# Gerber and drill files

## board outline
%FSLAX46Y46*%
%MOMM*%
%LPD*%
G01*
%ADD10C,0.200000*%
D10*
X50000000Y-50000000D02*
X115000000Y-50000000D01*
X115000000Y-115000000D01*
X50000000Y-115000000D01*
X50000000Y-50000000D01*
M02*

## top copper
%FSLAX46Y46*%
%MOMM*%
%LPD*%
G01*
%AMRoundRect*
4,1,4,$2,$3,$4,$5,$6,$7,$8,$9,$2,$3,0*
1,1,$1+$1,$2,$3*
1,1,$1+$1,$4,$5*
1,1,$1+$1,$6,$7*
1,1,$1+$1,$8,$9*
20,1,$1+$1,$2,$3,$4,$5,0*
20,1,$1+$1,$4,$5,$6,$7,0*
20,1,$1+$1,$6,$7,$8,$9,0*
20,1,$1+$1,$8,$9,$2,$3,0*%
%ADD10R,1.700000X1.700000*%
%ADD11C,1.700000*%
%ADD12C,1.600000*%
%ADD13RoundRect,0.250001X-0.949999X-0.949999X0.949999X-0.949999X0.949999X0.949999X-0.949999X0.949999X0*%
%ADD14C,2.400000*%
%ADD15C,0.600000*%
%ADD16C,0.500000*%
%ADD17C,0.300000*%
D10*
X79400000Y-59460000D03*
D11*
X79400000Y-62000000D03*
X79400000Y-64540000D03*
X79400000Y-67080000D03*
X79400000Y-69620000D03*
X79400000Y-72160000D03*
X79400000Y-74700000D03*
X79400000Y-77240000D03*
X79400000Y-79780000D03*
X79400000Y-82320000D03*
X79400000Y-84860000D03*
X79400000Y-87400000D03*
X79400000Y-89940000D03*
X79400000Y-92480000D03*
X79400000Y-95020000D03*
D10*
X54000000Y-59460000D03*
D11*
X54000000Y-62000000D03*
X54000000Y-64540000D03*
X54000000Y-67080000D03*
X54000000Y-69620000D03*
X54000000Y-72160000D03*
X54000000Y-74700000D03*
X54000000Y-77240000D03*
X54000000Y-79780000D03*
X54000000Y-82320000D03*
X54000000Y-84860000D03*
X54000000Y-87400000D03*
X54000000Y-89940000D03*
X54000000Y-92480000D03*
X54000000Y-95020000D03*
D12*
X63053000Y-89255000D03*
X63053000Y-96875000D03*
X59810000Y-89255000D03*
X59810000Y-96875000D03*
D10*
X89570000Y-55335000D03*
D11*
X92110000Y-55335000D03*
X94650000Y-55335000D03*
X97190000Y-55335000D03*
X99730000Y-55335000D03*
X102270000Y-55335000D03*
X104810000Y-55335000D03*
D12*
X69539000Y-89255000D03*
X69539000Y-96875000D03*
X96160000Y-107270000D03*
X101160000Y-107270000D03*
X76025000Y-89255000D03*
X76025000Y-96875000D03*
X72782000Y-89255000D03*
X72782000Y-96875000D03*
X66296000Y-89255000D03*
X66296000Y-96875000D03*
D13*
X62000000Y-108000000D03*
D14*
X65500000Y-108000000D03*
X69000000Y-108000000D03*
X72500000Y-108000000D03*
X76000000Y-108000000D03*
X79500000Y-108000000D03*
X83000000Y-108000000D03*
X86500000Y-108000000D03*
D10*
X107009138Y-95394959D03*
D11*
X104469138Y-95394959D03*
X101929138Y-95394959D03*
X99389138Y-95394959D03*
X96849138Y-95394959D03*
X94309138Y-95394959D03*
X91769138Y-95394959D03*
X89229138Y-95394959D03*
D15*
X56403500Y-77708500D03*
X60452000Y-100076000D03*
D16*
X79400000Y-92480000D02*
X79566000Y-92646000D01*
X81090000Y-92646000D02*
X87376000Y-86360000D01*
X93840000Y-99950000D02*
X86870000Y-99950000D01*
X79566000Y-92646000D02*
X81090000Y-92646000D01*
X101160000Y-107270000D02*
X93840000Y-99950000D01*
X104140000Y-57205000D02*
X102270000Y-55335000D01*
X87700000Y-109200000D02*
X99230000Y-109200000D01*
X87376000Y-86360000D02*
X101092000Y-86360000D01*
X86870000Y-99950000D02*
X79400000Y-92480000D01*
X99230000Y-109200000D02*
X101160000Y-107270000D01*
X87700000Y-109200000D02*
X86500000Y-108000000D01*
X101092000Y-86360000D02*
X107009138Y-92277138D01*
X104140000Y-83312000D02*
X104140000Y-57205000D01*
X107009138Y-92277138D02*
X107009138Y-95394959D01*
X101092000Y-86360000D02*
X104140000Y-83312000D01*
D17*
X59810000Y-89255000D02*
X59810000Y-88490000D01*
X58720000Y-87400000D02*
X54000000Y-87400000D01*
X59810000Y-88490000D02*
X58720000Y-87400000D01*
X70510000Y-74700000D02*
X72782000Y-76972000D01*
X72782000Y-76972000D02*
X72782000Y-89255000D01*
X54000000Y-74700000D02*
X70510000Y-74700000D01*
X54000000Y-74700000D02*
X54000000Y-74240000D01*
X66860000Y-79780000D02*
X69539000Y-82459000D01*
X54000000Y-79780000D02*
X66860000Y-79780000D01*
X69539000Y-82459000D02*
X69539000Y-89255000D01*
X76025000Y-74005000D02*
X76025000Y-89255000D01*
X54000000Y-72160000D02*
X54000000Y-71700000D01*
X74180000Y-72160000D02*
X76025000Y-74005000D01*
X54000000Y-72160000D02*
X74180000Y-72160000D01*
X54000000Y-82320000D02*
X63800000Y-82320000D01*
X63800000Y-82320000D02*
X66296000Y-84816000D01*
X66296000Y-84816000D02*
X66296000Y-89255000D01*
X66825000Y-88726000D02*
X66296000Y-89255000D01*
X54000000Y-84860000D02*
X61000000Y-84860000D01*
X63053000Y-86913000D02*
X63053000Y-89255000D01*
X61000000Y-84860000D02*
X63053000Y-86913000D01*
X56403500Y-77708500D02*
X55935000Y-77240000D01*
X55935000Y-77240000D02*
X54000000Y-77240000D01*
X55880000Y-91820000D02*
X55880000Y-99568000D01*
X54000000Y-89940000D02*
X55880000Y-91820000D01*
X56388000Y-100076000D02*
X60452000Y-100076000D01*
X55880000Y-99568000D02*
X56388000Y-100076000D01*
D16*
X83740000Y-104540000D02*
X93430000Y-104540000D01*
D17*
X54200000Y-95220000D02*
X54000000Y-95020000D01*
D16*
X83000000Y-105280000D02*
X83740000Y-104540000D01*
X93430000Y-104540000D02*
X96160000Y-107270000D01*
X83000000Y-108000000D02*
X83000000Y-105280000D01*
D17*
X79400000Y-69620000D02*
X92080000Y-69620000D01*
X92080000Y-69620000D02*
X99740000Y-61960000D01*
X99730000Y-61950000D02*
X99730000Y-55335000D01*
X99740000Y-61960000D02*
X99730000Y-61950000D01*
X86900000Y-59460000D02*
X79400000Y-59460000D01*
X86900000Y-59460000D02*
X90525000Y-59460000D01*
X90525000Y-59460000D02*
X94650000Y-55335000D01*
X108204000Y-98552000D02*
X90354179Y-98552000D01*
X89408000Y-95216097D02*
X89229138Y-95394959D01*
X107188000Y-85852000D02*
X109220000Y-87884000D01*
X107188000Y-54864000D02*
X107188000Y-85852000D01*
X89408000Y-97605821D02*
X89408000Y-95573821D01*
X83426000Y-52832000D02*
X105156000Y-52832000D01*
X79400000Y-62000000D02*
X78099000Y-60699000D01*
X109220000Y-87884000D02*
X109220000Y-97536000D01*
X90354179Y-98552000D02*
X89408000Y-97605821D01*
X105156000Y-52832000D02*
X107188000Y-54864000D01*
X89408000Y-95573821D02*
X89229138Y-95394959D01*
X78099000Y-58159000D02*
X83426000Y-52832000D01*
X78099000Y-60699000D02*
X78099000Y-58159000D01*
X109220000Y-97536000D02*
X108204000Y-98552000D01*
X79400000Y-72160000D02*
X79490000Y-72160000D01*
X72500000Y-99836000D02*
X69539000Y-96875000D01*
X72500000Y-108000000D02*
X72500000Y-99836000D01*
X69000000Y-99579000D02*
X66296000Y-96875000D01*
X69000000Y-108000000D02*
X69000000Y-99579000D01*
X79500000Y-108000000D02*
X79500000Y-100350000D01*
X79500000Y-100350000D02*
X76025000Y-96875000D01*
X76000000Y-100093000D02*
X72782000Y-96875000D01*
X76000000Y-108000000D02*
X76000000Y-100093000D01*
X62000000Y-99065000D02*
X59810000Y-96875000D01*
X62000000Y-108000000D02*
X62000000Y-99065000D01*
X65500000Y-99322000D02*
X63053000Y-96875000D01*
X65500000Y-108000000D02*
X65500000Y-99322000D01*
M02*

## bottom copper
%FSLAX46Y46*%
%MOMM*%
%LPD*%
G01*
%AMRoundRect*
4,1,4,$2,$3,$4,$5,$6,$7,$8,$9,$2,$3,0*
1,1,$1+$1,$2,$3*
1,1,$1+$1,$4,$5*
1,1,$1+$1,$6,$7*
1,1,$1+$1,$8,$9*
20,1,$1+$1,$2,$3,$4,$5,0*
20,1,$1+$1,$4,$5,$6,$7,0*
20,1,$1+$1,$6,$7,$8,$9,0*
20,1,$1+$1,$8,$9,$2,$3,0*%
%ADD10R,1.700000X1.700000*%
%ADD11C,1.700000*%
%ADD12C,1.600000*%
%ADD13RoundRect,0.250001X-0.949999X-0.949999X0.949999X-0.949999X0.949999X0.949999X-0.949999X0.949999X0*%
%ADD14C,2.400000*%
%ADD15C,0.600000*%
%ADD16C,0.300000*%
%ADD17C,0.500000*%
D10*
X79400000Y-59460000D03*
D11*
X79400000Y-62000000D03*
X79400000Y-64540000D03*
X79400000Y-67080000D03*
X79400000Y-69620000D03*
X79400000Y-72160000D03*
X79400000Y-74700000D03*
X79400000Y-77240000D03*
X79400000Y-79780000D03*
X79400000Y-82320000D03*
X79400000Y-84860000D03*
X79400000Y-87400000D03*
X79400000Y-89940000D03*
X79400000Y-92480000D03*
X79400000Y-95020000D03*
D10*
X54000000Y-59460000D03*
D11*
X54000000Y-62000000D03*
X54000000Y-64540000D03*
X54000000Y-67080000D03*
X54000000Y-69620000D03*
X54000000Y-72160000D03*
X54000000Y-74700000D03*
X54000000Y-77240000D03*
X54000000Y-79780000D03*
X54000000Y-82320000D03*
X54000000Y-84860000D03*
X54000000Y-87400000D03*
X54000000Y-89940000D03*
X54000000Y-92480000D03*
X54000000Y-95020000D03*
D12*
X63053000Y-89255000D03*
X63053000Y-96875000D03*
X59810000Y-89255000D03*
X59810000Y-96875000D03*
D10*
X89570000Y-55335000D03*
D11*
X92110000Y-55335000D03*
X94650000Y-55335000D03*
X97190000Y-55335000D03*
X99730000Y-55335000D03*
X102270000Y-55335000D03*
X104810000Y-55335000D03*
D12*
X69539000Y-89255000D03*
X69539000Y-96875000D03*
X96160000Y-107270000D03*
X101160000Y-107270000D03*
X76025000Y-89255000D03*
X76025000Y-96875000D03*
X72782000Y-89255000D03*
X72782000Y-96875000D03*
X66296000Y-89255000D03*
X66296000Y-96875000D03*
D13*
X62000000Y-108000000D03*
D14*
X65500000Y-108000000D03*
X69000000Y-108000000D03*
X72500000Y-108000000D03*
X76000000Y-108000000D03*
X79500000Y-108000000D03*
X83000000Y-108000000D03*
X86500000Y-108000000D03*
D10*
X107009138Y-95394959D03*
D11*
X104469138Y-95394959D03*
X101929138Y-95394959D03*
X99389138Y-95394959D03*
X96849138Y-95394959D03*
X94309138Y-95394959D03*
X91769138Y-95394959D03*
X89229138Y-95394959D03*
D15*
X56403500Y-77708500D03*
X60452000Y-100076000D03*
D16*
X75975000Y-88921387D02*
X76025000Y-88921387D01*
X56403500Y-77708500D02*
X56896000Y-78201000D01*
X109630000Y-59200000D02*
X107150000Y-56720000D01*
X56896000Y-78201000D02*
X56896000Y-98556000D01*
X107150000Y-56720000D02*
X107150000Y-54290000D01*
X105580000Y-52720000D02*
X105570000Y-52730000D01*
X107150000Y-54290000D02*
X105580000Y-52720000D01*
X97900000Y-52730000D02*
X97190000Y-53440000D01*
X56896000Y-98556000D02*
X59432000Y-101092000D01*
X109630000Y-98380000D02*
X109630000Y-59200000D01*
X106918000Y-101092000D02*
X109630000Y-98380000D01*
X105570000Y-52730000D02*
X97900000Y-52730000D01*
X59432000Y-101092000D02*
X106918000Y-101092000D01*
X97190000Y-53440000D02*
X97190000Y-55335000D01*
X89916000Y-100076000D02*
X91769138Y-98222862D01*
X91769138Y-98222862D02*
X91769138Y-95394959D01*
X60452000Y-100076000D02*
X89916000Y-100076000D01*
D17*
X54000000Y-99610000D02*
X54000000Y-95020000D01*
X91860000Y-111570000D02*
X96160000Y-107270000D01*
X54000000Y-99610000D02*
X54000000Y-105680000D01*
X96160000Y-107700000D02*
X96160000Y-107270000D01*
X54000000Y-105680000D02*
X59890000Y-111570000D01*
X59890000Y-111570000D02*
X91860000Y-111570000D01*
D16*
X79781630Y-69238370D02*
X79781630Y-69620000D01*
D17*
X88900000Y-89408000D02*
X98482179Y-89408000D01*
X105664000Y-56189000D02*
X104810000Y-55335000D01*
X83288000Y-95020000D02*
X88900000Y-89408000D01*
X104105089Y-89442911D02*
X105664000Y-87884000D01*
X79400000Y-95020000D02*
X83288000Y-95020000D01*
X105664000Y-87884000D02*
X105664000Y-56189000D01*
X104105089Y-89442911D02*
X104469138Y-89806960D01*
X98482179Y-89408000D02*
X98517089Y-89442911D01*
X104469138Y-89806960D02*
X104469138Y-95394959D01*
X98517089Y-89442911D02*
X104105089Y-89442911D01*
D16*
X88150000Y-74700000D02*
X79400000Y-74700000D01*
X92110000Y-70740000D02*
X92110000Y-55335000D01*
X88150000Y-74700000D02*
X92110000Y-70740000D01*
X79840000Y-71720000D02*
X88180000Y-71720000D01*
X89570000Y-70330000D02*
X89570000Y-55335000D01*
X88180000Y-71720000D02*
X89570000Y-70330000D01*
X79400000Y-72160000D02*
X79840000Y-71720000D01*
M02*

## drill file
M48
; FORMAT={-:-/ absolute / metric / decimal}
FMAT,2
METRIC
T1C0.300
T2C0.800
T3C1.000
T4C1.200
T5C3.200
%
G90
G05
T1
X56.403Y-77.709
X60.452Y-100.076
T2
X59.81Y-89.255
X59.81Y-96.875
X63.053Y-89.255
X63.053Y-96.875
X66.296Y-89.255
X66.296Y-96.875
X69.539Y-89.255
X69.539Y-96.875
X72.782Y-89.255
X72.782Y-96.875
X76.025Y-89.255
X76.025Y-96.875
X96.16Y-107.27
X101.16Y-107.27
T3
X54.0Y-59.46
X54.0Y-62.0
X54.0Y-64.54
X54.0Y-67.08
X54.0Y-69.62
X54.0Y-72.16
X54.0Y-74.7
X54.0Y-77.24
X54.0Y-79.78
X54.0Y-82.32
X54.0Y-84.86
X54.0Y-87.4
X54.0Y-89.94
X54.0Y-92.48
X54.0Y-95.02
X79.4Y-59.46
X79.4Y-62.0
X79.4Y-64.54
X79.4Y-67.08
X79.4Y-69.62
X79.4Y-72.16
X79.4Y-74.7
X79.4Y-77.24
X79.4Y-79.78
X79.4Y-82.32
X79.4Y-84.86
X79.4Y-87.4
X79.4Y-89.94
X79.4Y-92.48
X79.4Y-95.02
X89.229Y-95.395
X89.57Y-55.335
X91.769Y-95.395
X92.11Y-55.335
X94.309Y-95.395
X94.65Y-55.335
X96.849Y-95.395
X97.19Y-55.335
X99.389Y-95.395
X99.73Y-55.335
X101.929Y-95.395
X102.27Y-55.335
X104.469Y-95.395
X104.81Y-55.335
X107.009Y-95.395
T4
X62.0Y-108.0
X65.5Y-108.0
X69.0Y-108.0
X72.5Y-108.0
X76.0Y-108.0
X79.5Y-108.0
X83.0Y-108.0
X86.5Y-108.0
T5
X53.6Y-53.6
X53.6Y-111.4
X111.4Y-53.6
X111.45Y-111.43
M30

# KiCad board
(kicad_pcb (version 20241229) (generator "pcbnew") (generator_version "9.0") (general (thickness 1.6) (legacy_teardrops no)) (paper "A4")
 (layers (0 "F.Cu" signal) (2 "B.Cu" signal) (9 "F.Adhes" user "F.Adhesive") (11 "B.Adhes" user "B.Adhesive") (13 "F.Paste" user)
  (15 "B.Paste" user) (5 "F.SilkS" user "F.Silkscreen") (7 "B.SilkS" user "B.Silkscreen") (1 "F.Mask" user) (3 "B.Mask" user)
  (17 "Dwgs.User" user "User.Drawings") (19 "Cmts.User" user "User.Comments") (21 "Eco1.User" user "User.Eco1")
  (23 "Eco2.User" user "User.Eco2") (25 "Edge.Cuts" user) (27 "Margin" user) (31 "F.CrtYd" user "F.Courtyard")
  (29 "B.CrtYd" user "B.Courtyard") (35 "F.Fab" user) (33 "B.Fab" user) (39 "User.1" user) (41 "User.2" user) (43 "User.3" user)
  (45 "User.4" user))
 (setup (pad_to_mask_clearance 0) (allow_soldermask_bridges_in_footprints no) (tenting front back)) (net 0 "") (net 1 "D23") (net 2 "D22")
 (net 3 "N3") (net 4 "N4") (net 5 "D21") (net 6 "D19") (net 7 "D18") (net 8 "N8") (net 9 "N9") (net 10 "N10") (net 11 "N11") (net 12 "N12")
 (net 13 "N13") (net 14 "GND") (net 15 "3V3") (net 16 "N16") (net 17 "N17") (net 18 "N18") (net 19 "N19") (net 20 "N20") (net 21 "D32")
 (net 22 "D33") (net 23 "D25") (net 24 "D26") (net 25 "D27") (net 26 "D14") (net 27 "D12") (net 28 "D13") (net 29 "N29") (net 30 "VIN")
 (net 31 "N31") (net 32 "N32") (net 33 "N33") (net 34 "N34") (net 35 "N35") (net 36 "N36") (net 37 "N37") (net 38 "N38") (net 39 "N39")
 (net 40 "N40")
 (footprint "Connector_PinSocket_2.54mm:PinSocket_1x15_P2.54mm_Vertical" (layer "F.Cu") (at 79.4 59.46)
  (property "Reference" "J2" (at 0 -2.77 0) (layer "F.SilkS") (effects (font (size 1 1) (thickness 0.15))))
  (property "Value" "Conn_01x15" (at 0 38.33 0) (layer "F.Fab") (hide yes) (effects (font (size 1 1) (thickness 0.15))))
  (pad "1" thru_hole rect (at 0 0) (size 1.7 1.7) (drill 1) (layers "*.Cu" "*.Mask") (remove_unused_layers no) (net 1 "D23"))
  (pad "2" thru_hole circle (at 0 2.54) (size 1.7 1.7) (drill 1) (layers "*.Cu" "*.Mask") (remove_unused_layers no) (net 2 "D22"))
  (pad "3" thru_hole circle (at 0 5.08) (size 1.7 1.7) (drill 1) (layers "*.Cu" "*.Mask") (remove_unused_layers no) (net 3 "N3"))
  (pad "4" thru_hole circle (at 0 7.62) (size 1.7 1.7) (drill 1) (layers "*.Cu" "*.Mask") (remove_unused_layers no) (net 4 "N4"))
  (pad "5" thru_hole circle (at 0 10.16) (size 1.7 1.7) (drill 1) (layers "*.Cu" "*.Mask") (remove_unused_layers no) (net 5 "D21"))
  (pad "6" thru_hole circle (at 0 12.7) (size 1.7 1.7) (drill 1) (layers "*.Cu" "*.Mask") (remove_unused_layers no) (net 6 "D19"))
  (pad "7" thru_hole circle (at 0 15.24) (size 1.7 1.7) (drill 1) (layers "*.Cu" "*.Mask") (remove_unused_layers no) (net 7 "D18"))
  (pad "8" thru_hole circle (at 0 17.78) (size 1.7 1.7) (drill 1) (layers "*.Cu" "*.Mask") (remove_unused_layers no) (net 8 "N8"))
  (pad "9" thru_hole circle (at 0 20.32) (size 1.7 1.7) (drill 1) (layers "*.Cu" "*.Mask") (remove_unused_layers no) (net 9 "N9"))
  (pad "10" thru_hole circle (at 0 22.86) (size 1.7 1.7) (drill 1) (layers "*.Cu" "*.Mask") (remove_unused_layers no) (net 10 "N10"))
  (pad "11" thru_hole circle (at 0 25.4) (size 1.7 1.7) (drill 1) (layers "*.Cu" "*.Mask") (remove_unused_layers no) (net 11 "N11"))
  (pad "12" thru_hole circle (at 0 27.94) (size 1.7 1.7) (drill 1) (layers "*.Cu" "*.Mask") (remove_unused_layers no) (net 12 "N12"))
  (pad "13" thru_hole circle (at 0 30.48) (size 1.7 1.7) (drill 1) (layers "*.Cu" "*.Mask") (remove_unused_layers no) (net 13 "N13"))
  (pad "14" thru_hole circle (at 0 33.02) (size 1.7 1.7) (drill 1) (layers "*.Cu" "*.Mask") (remove_unused_layers no) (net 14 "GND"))
  (pad "15" thru_hole circle (at 0 35.56) (size 1.7 1.7) (drill 1) (layers "*.Cu" "*.Mask") (remove_unused_layers no) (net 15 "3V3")))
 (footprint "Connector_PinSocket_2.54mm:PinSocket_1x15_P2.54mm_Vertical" (layer "F.Cu") (at 54 59.46)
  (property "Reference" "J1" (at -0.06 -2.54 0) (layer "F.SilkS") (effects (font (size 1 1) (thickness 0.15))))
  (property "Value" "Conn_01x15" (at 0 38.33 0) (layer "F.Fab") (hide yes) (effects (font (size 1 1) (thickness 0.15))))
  (pad "1" thru_hole rect (at 0 0) (size 1.7 1.7) (drill 1) (layers "*.Cu" "*.Mask") (remove_unused_layers no) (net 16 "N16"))
  (pad "2" thru_hole circle (at 0 2.54) (size 1.7 1.7) (drill 1) (layers "*.Cu" "*.Mask") (remove_unused_layers no) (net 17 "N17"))
  (pad "3" thru_hole circle (at 0 5.08) (size 1.7 1.7) (drill 1) (layers "*.Cu" "*.Mask") (remove_unused_layers no) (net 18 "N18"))
  (pad "4" thru_hole circle (at 0 7.62) (size 1.7 1.7) (drill 1) (layers "*.Cu" "*.Mask") (remove_unused_layers no) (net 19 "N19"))
  (pad "5" thru_hole circle (at 0 10.16) (size 1.7 1.7) (drill 1) (layers "*.Cu" "*.Mask") (remove_unused_layers no) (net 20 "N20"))
  (pad "6" thru_hole circle (at 0 12.7) (size 1.7 1.7) (drill 1) (layers "*.Cu" "*.Mask") (remove_unused_layers no) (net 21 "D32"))
  (pad "7" thru_hole circle (at 0 15.24) (size 1.7 1.7) (drill 1) (layers "*.Cu" "*.Mask") (remove_unused_layers no) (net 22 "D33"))
  (pad "8" thru_hole circle (at 0 17.78) (size 1.7 1.7) (drill 1) (layers "*.Cu" "*.Mask") (remove_unused_layers no) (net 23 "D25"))
  (pad "9" thru_hole circle (at 0 20.32) (size 1.7 1.7) (drill 1) (layers "*.Cu" "*.Mask") (remove_unused_layers no) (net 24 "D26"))
  (pad "10" thru_hole circle (at 0 22.86) (size 1.7 1.7) (drill 1) (layers "*.Cu" "*.Mask") (remove_unused_layers no) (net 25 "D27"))
  (pad "11" thru_hole circle (at 0 25.4) (size 1.7 1.7) (drill 1) (layers "*.Cu" "*.Mask") (remove_unused_layers no) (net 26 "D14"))
  (pad "12" thru_hole circle (at 0 27.94) (size 1.7 1.7) (drill 1) (layers "*.Cu" "*.Mask") (remove_unused_layers no) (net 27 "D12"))
  (pad "13" thru_hole circle (at 0 30.48) (size 1.7 1.7) (drill 1) (layers "*.Cu" "*.Mask") (remove_unused_layers no) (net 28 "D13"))
  (pad "14" thru_hole circle (at 0 33.02) (size 1.7 1.7) (drill 1) (layers "*.Cu" "*.Mask") (remove_unused_layers no) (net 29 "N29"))
  (pad "15" thru_hole circle (at 0 35.56) (size 1.7 1.7) (drill 1) (layers "*.Cu" "*.Mask") (remove_unused_layers no) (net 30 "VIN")))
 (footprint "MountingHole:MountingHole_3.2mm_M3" (layer "F.Cu") (at 53.6 53.6)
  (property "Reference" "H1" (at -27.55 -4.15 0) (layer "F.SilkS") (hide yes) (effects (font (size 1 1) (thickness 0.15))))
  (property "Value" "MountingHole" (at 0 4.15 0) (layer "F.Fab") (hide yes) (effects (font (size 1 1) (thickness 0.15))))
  (pad "" np_thru_hole circle (at 0 0) (size 3.2 3.2) (drill 3.2) (layers "*.Cu" "*.Mask")))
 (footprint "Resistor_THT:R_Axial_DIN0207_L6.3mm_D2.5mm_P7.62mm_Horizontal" (layer "F.Cu") (at 63.053 89.255 -90)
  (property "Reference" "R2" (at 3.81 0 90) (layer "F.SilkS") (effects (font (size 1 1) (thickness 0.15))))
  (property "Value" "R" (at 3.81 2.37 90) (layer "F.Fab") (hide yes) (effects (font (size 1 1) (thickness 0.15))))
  (pad "1" thru_hole circle (at 0 0 270) (size 1.6 1.6) (drill 0.8) (layers "*.Cu" "*.Mask") (remove_unused_layers no) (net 26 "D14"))
  (pad "2" thru_hole circle (at 7.62 0 270) (size 1.6 1.6) (drill 0.8) (layers "*.Cu" "*.Mask") (remove_unused_layers no) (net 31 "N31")))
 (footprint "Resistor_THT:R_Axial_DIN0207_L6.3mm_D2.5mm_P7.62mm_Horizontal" (layer "F.Cu") (at 59.81 89.255 -90)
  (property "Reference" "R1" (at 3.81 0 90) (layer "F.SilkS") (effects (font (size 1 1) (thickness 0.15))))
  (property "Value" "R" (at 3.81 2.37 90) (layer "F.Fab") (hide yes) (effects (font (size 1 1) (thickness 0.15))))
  (pad "1" thru_hole circle (at 0 0 270) (size 1.6 1.6) (drill 0.8) (layers "*.Cu" "*.Mask") (remove_unused_layers no) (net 27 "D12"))
  (pad "2" thru_hole circle (at 7.62 0 270) (size 1.6 1.6) (drill 0.8) (layers "*.Cu" "*.Mask") (remove_unused_layers no) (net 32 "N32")))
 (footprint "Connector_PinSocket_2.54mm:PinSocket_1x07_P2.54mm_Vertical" (layer "F.Cu") (at 89.57 55.335 90)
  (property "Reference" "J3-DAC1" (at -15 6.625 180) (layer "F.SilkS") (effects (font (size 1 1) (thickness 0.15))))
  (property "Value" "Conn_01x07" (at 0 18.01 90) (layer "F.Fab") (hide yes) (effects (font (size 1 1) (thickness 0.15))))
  (pad "1" thru_hole rect (at 0 0 90) (size 1.7 1.7) (drill 1) (layers "*.Cu" "*.Mask") (remove_unused_layers no) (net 6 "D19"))
  (pad "2" thru_hole circle (at 0 2.54 90) (size 1.7 1.7) (drill 1) (layers "*.Cu" "*.Mask") (remove_unused_layers no) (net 7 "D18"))
  (pad "3" thru_hole circle (at 0 5.08 90) (size 1.7 1.7) (drill 1) (layers "*.Cu" "*.Mask") (remove_unused_layers no) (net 1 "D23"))
  (pad "4" thru_hole circle (at 0 7.62 90) (size 1.7 1.7) (drill 1) (layers "*.Cu" "*.Mask") (remove_unused_layers no) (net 23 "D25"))
  (pad "5" thru_hole circle (at 0 10.16 90) (size 1.7 1.7) (drill 1) (layers "*.Cu" "*.Mask") (remove_unused_layers no) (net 5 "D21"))
  (pad "6" thru_hole circle (at 0 12.7 90) (size 1.7 1.7) (drill 1) (layers "*.Cu" "*.Mask") (remove_unused_layers no) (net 14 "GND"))
  (pad "7" thru_hole circle (at 0 15.24 90) (size 1.7 1.7) (drill 1) (layers "*.Cu" "*.Mask") (remove_unused_layers no) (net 15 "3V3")))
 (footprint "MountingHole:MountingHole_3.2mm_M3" (layer "F.Cu") (at 53.6 111.4)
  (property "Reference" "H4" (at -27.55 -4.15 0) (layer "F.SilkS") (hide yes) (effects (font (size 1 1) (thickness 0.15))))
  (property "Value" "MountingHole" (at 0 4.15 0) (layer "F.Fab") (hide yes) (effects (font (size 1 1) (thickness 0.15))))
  (pad "" np_thru_hole circle (at 0 0) (size 3.2 3.2) (drill 3.2) (layers "*.Cu" "*.Mask")))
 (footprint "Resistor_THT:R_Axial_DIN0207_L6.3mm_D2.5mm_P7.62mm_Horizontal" (layer "F.Cu") (at 69.539 89.255 -90)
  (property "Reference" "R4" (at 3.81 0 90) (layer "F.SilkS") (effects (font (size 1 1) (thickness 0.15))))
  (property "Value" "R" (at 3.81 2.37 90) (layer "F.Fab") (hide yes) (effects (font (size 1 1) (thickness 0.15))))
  (pad "1" thru_hole circle (at 0 0 270) (size 1.6 1.6) (drill 0.8) (layers "*.Cu" "*.Mask") (remove_unused_layers no) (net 24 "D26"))
  (pad "2" thru_hole circle (at 7.62 0 270) (size 1.6 1.6) (drill 0.8) (layers "*.Cu" "*.Mask") (remove_unused_layers no) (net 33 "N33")))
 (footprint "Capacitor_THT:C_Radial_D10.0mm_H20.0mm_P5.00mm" (layer "F.Cu") (at 96.16 107.27)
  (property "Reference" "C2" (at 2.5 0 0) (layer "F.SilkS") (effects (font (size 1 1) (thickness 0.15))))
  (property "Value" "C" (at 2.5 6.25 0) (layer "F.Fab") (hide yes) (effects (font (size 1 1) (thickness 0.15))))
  (pad "1" thru_hole circle (at 0 0) (size 1.6 1.6) (drill 0.8) (layers "*.Cu" "*.Mask") (remove_unused_layers no) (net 30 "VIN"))
  (pad "2" thru_hole circle (at 5 0) (size 1.6 1.6) (drill 0.8) (layers "*.Cu" "*.Mask") (remove_unused_layers no) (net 14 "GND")))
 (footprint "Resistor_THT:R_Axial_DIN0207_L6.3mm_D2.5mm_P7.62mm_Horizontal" (layer "F.Cu") (at 76.025 89.255 -90)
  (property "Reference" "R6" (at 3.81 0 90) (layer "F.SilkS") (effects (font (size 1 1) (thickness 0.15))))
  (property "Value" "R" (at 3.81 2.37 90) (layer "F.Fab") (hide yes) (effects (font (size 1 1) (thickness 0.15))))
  (pad "1" thru_hole circle (at 0 0 270) (size 1.6 1.6) (drill 0.8) (layers "*.Cu" "*.Mask") (remove_unused_layers no) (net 21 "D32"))
  (pad "2" thru_hole circle (at 7.62 0 270) (size 1.6 1.6) (drill 0.8) (layers "*.Cu" "*.Mask") (remove_unused_layers no) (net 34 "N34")))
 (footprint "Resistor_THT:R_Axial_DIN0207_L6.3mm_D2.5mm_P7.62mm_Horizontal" (layer "F.Cu") (at 72.782 89.255 -90)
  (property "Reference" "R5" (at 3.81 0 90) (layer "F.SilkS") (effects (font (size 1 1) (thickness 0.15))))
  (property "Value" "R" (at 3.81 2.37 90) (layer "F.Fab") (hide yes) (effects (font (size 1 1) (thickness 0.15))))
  (pad "1" thru_hole circle (at 0 0 270) (size 1.6 1.6) (drill 0.8) (layers "*.Cu" "*.Mask") (remove_unused_layers no) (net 22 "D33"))
  (pad "2" thru_hole circle (at 7.62 0 270) (size 1.6 1.6) (drill 0.8) (layers "*.Cu" "*.Mask") (remove_unused_layers no) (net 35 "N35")))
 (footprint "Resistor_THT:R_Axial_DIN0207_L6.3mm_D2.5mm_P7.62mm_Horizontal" (layer "F.Cu") (at 66.296 89.255 -90)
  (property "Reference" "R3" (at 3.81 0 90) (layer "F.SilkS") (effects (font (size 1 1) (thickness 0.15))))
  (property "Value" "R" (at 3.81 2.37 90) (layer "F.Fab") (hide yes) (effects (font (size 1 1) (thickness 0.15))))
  (pad "1" thru_hole circle (at 0 0 270) (size 1.6 1.6) (drill 0.8) (layers "*.Cu" "*.Mask") (remove_unused_layers no) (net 25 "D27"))
  (pad "2" thru_hole circle (at 7.62 0 270) (size 1.6 1.6) (drill 0.8) (layers "*.Cu" "*.Mask") (remove_unused_layers no) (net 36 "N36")))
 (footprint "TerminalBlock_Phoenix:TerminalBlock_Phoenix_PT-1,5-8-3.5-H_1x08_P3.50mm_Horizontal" (layer "F.Cu") (at 62 108)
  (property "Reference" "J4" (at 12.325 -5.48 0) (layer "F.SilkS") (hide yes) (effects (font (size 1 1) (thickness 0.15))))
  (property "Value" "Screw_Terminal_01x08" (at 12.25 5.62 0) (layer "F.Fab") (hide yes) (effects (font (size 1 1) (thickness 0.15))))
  (pad "1" thru_hole roundrect (at 0 0) (size 2.4 2.4) (drill 1.2) (layers "*.Cu" "*.Mask") (remove_unused_layers no)
   (roundrect_rratio 0.104167) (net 32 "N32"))
  (pad "2" thru_hole circle (at 3.5 0) (size 2.4 2.4) (drill 1.2) (layers "*.Cu" "*.Mask") (remove_unused_layers no) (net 31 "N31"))
  (pad "3" thru_hole circle (at 7 0) (size 2.4 2.4) (drill 1.2) (layers "*.Cu" "*.Mask") (remove_unused_layers no) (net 36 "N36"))
  (pad "4" thru_hole circle (at 10.5 0) (size 2.4 2.4) (drill 1.2) (layers "*.Cu" "*.Mask") (remove_unused_layers no) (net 33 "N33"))
  (pad "5" thru_hole circle (at 14 0) (size 2.4 2.4) (drill 1.2) (layers "*.Cu" "*.Mask") (remove_unused_layers no) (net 35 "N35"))
  (pad "6" thru_hole circle (at 17.5 0) (size 2.4 2.4) (drill 1.2) (layers "*.Cu" "*.Mask") (remove_unused_layers no) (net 34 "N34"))
  (pad "7" thru_hole circle (at 21 0) (size 2.4 2.4) (drill 1.2) (layers "*.Cu" "*.Mask") (remove_unused_layers no) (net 30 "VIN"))
  (pad "8" thru_hole circle (at 24.5 0) (size 2.4 2.4) (drill 1.2) (layers "*.Cu" "*.Mask") (remove_unused_layers no) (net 14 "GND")))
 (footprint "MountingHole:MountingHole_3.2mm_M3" (layer "F.Cu") (at 111.45 111.43)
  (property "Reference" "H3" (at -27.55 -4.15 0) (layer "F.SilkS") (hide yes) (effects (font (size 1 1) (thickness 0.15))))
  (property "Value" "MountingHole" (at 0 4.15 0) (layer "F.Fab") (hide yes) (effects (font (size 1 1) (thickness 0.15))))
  (pad "" np_thru_hole circle (at 0 0) (size 3.2 3.2) (drill 3.2) (layers "*.Cu" "*.Mask")))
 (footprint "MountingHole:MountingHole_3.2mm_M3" (layer "F.Cu") (at 111.4 53.6)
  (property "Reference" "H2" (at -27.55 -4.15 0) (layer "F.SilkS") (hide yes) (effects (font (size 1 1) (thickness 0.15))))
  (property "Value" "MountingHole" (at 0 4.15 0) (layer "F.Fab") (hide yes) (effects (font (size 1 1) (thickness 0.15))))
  (pad "" np_thru_hole circle (at 0 0) (size 3.2 3.2) (drill 3.2) (layers "*.Cu" "*.Mask")))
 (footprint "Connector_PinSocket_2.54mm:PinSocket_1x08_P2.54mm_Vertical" (layer "F.Cu") (at 107.009138 95.394959 -90)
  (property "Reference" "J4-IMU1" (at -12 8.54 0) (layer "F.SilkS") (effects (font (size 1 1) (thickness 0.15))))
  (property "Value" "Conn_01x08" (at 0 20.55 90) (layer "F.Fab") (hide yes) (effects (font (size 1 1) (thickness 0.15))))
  (pad "1" thru_hole rect (at 0 0 270) (size 1.7 1.7) (drill 1) (layers "*.Cu" "*.Mask") (remove_unused_layers no) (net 14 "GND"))
  (pad "2" thru_hole circle (at 0 2.54 270) (size 1.7 1.7) (drill 1) (layers "*.Cu" "*.Mask") (remove_unused_layers no) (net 15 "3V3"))
  (pad "3" thru_hole circle (at 0 5.08 270) (size 1.7 1.7) (drill 1) (layers "*.Cu" "*.Mask") (remove_unused_layers no) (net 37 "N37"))
  (pad "4" thru_hole circle (at 0 7.62 270) (size 1.7 1.7) (drill 1) (layers "*.Cu" "*.Mask") (remove_unused_layers no) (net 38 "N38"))
  (pad "5" thru_hole circle (at 0 10.16 270) (size 1.7 1.7) (drill 1) (layers "*.Cu" "*.Mask") (remove_unused_layers no) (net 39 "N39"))
  (pad "6" thru_hole circle (at 0 12.7 270) (size 1.7 1.7) (drill 1) (layers "*.Cu" "*.Mask") (remove_unused_layers no) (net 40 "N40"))
  (pad "7" thru_hole circle (at 0 15.24 270) (size 1.7 1.7) (drill 1) (layers "*.Cu" "*.Mask") (remove_unused_layers no) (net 28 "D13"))
  (pad "8" thru_hole circle (at 0 17.78 270) (size 1.7 1.7) (drill 1) (layers "*.Cu" "*.Mask") (remove_unused_layers no) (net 2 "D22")))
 (gr_rect (start 50 50) (end 115 115) (stroke (width 0.2) (type solid)) (fill no) (layer "Edge.Cuts"))
 (segment (start 79.4 92.48) (end 79.566 92.646) (width 0.5) (layer "F.Cu") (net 14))
 (segment (start 81.09 92.646) (end 87.376 86.36) (width 0.5) (layer "F.Cu") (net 14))
 (segment (start 93.84 99.95) (end 86.87 99.95) (width 0.5) (layer "F.Cu") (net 14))
 (segment (start 79.566 92.646) (end 81.09 92.646) (width 0.5) (layer "F.Cu") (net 14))
 (segment (start 101.16 107.27) (end 93.84 99.95) (width 0.5) (layer "F.Cu") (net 14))
 (segment (start 104.14 57.205) (end 102.27 55.335) (width 0.5) (layer "F.Cu") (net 14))
 (segment (start 87.7 109.2) (end 99.23 109.2) (width 0.5) (layer "F.Cu") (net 14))
 (segment (start 87.376 86.36) (end 101.092 86.36) (width 0.5) (layer "F.Cu") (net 14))
 (segment (start 86.87 99.95) (end 79.4 92.48) (width 0.5) (layer "F.Cu") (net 14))
 (segment (start 99.23 109.2) (end 101.16 107.27) (width 0.5) (layer "F.Cu") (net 14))
 (segment (start 87.7 109.2) (end 86.5 108) (width 0.5) (layer "F.Cu") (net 14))
 (segment (start 101.092 86.36) (end 107.009138 92.277138) (width 0.5) (layer "F.Cu") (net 14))
 (segment (start 104.14 83.312) (end 104.14 57.205) (width 0.5) (layer "F.Cu") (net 14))
 (segment (start 107.009138 92.277138) (end 107.009138 95.394959) (width 0.5) (layer "F.Cu") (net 14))
 (segment (start 101.092 86.36) (end 104.14 83.312) (width 0.5) (layer "F.Cu") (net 14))
 (segment (start 59.81 89.255) (end 59.81 88.49) (width 0.3) (layer "F.Cu") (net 27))
 (segment (start 58.72 87.4) (end 54 87.4) (width 0.3) (layer "F.Cu") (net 27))
 (segment (start 59.81 88.49) (end 58.72 87.4) (width 0.3) (layer "F.Cu") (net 27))
 (segment (start 70.51 74.7) (end 72.782 76.972) (width 0.3) (layer "F.Cu") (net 22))
 (segment (start 72.782 76.972) (end 72.782 89.255) (width 0.3) (layer "F.Cu") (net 22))
 (segment (start 54 74.7) (end 70.51 74.7) (width 0.3) (layer "F.Cu") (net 22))
 (segment (start 54 74.7) (end 54 74.24) (width 0.3) (layer "F.Cu") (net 22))
 (segment (start 66.86 79.78) (end 69.539 82.459) (width 0.3) (layer "F.Cu") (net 24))
 (segment (start 54 79.78) (end 66.86 79.78) (width 0.3) (layer "F.Cu") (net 24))
 (segment (start 69.539 82.459) (end 69.539 89.255) (width 0.3) (layer "F.Cu") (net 24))
 (segment (start 76.025 74.005) (end 76.025 89.255) (width 0.3) (layer "F.Cu") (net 21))
 (segment (start 54 72.16) (end 54 71.7) (width 0.3) (layer "F.Cu") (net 21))
 (segment (start 74.18 72.16) (end 76.025 74.005) (width 0.3) (layer "F.Cu") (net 21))
 (segment (start 54 72.16) (end 74.18 72.16) (width 0.3) (layer "F.Cu") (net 21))
 (segment (start 75.975 88.921387) (end 76.025 88.921387) (width 0.3) (layer "B.Cu") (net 21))
 (segment (start 54 82.32) (end 63.8 82.32) (width 0.3) (layer "F.Cu") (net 25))
 (segment (start 63.8 82.32) (end 66.296 84.816) (width 0.3) (layer "F.Cu") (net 25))
 (segment (start 66.296 84.816) (end 66.296 89.255) (width 0.3) (layer "F.Cu") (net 25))
 (segment (start 66.825 88.726) (end 66.296 89.255) (width 0.3) (layer "F.Cu") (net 25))
 (segment (start 54 84.86) (end 61 84.86) (width 0.3) (layer "F.Cu") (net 26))
 (segment (start 63.053 86.913) (end 63.053 89.255) (width 0.3) (layer "F.Cu") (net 26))
 (segment (start 61 84.86) (end 63.053 86.913) (width 0.3) (layer "F.Cu") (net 26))
 (segment (start 56.4035 77.7085) (end 55.935 77.24) (width 0.3) (layer "F.Cu") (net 23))
 (segment (start 55.935 77.24) (end 54 77.24) (width 0.3) (layer "F.Cu") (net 23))
 (via (at 56.4035 77.7085) (size 0.6) (drill 0.3) (layers "F.Cu" "B.Cu") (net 23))
 (segment (start 56.4035 77.7085) (end 56.896 78.201) (width 0.3) (layer "B.Cu") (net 23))
 (segment (start 109.63 59.2) (end 107.15 56.72) (width 0.3) (layer "B.Cu") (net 23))
 (segment (start 56.896 78.201) (end 56.896 98.556) (width 0.3) (layer "B.Cu") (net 23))
 (segment (start 107.15 56.72) (end 107.15 54.29) (width 0.3) (layer "B.Cu") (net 23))
 (segment (start 105.58 52.72) (end 105.57 52.73) (width 0.3) (layer "B.Cu") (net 23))
 (segment (start 107.15 54.29) (end 105.58 52.72) (width 0.3) (layer "B.Cu") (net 23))
 (segment (start 97.9 52.73) (end 97.19 53.44) (width 0.3) (layer "B.Cu") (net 23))
 (segment (start 56.896 98.556) (end 59.432 101.092) (width 0.3) (layer "B.Cu") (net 23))
 (segment (start 109.63 98.38) (end 109.63 59.2) (width 0.3) (layer "B.Cu") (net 23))
 (segment (start 106.918 101.092) (end 109.63 98.38) (width 0.3) (layer "B.Cu") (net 23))
 (segment (start 105.57 52.73) (end 97.9 52.73) (width 0.3) (layer "B.Cu") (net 23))
 (segment (start 59.432 101.092) (end 106.918 101.092) (width 0.3) (layer "B.Cu") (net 23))
 (segment (start 97.19 53.44) (end 97.19 55.335) (width 0.3) (layer "B.Cu") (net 23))
 (segment (start 55.88 91.82) (end 55.88 99.568) (width 0.3) (layer "F.Cu") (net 28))
 (segment (start 54 89.94) (end 55.88 91.82) (width 0.3) (layer "F.Cu") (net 28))
 (segment (start 56.388 100.076) (end 60.452 100.076) (width 0.3) (layer "F.Cu") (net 28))
 (segment (start 55.88 99.568) (end 56.388 100.076) (width 0.3) (layer "F.Cu") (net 28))
 (via (at 60.452 100.076) (size 0.6) (drill 0.3) (layers "F.Cu" "B.Cu") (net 28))
 (segment (start 89.916 100.076) (end 91.769138 98.222862) (width 0.3) (layer "B.Cu") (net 28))
 (segment (start 91.769138 98.222862) (end 91.769138 95.394959) (width 0.3) (layer "B.Cu") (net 28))
 (segment (start 60.452 100.076) (end 89.916 100.076) (width 0.3) (layer "B.Cu") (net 28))
 (segment (start 83.74 104.54) (end 93.43 104.54) (width 0.5) (layer "F.Cu") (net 30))
 (segment (start 54.2 95.22) (end 54 95.02) (width 0.3) (layer "F.Cu") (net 30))
 (segment (start 83 105.28) (end 83.74 104.54) (width 0.5) (layer "F.Cu") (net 30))
 (segment (start 93.43 104.54) (end 96.16 107.27) (width 0.5) (layer "F.Cu") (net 30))
 (segment (start 83 108) (end 83 105.28) (width 0.5) (layer "F.Cu") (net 30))
 (segment (start 54 99.61) (end 54 95.02) (width 0.5) (layer "B.Cu") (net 30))
 (segment (start 91.86 111.57) (end 96.16 107.27) (width 0.5) (layer "B.Cu") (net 30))
 (segment (start 54 99.61) (end 54 105.68) (width 0.5) (layer "B.Cu") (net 30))
 (segment (start 96.16 107.7) (end 96.16 107.27) (width 0.5) (layer "B.Cu") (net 30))
 (segment (start 54 105.68) (end 59.89 111.57) (width 0.5) (layer "B.Cu") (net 30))
 (segment (start 59.89 111.57) (end 91.86 111.57) (width 0.5) (layer "B.Cu") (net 30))
 (segment (start 79.4 69.62) (end 92.08 69.62) (width 0.3) (layer "F.Cu") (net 5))
 (segment (start 92.08 69.62) (end 99.74 61.96) (width 0.3) (layer "F.Cu") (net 5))
 (segment (start 99.73 61.95) (end 99.73 55.335) (width 0.3) (layer "F.Cu") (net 5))
 (segment (start 99.74 61.96) (end 99.73 61.95) (width 0.3) (layer "F.Cu") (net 5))
 (segment (start 79.78163 69.23837) (end 79.78163 69.62) (width 0.3) (layer "B.Cu") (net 5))
 (segment (start 86.9 59.46) (end 79.4 59.46) (width 0.3) (layer "F.Cu") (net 1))
 (segment (start 86.9 59.46) (end 90.525 59.46) (width 0.3) (layer "F.Cu") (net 1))
 (segment (start 90.525 59.46) (end 94.65 55.335) (width 0.3) (layer "F.Cu") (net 1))
 (segment (start 108.204 98.552) (end 90.354179 98.552) (width 0.3) (layer "F.Cu") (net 2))
 (segment (start 89.408 95.216097) (end 89.229138 95.394959) (width 0.3) (layer "F.Cu") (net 2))
 (segment (start 107.188 85.852) (end 109.22 87.884) (width 0.3) (layer "F.Cu") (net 2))
 (segment (start 107.188 54.864) (end 107.188 85.852) (width 0.3) (layer "F.Cu") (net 2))
 (segment (start 89.408 97.605821) (end 89.408 95.573821) (width 0.3) (layer "F.Cu") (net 2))
 (segment (start 83.426 52.832) (end 105.156 52.832) (width 0.3) (layer "F.Cu") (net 2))
 (segment (start 79.4 62) (end 78.099 60.699) (width 0.3) (layer "F.Cu") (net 2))
 (segment (start 109.22 87.884) (end 109.22 97.536) (width 0.3) (layer "F.Cu") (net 2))
 (segment (start 90.354179 98.552) (end 89.408 97.605821) (width 0.3) (layer "F.Cu") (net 2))
 (segment (start 105.156 52.832) (end 107.188 54.864) (width 0.3) (layer "F.Cu") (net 2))
 (segment (start 89.408 95.573821) (end 89.229138 95.394959) (width 0.3) (layer "F.Cu") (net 2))
 (segment (start 78.099 58.159) (end 83.426 52.832) (width 0.3) (layer "F.Cu") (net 2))
 (segment (start 78.099 60.699) (end 78.099 58.159) (width 0.3) (layer "F.Cu") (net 2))
 (segment (start 109.22 97.536) (end 108.204 98.552) (width 0.3) (layer "F.Cu") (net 2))
 (segment (start 88.9 89.408) (end 98.482179 89.408) (width 0.5) (layer "B.Cu") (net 15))
 (segment (start 105.664 56.189) (end 104.81 55.335) (width 0.5) (layer "B.Cu") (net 15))
 (segment (start 83.288 95.02) (end 88.9 89.408) (width 0.5) (layer "B.Cu") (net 15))
 (segment (start 104.105089 89.442911) (end 105.664 87.884) (width 0.5) (layer "B.Cu") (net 15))
 (segment (start 79.4 95.02) (end 83.288 95.02) (width 0.5) (layer "B.Cu") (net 15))
 (segment (start 105.664 87.884) (end 105.664 56.189) (width 0.5) (layer "B.Cu") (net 15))
 (segment (start 104.105089 89.442911) (end 104.469138 89.80696) (width 0.5) (layer "B.Cu") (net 15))
 (segment (start 98.482179 89.408) (end 98.517089 89.442911) (width 0.5) (layer "B.Cu") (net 15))
 (segment (start 104.469138 89.80696) (end 104.469138 95.394959) (width 0.5) (layer "B.Cu") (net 15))
 (segment (start 98.517089 89.442911) (end 104.105089 89.442911) (width 0.5) (layer "B.Cu") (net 15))
 (segment (start 88.15 74.7) (end 79.4 74.7) (width 0.3) (layer "B.Cu") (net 7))
 (segment (start 92.11 70.74) (end 92.11 55.335) (width 0.3) (layer "B.Cu") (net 7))
 (segment (start 88.15 74.7) (end 92.11 70.74) (width 0.3) (layer "B.Cu") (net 7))
 (segment (start 79.4 72.16) (end 79.49 72.16) (width 0.3) (layer "F.Cu") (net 6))
 (segment (start 79.84 71.72) (end 88.18 71.72) (width 0.3) (layer "B.Cu") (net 6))
 (segment (start 89.57 70.33) (end 89.57 55.335) (width 0.3) (layer "B.Cu") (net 6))
 (segment (start 88.18 71.72) (end 89.57 70.33) (width 0.3) (layer "B.Cu") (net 6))
 (segment (start 79.4 72.16) (end 79.84 71.72) (width 0.3) (layer "B.Cu") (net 6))
 (segment (start 72.5 99.836) (end 69.539 96.875) (width 0.3) (layer "F.Cu") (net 33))
 (segment (start 72.5 108) (end 72.5 99.836) (width 0.3) (layer "F.Cu") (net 33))
 (segment (start 69 99.579) (end 66.296 96.875) (width 0.3) (layer "F.Cu") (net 36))
 (segment (start 69 108) (end 69 99.579) (width 0.3) (layer "F.Cu") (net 36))
 (segment (start 79.5 108) (end 79.5 100.35) (width 0.3) (layer "F.Cu") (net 34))
 (segment (start 79.5 100.35) (end 76.025 96.875) (width 0.3) (layer "F.Cu") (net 34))
 (segment (start 76 100.093) (end 72.782 96.875) (width 0.3) (layer "F.Cu") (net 35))
 (segment (start 76 108) (end 76 100.093) (width 0.3) (layer "F.Cu") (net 35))
 (segment (start 62 99.065) (end 59.81 96.875) (width 0.3) (layer "F.Cu") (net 32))
 (segment (start 62 108) (end 62 99.065) (width 0.3) (layer "F.Cu") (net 32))
 (segment (start 65.5 99.322) (end 63.053 96.875) (width 0.3) (layer "F.Cu") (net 31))
 (segment (start 65.5 108) (end 65.5 99.322) (width 0.3) (layer "F.Cu") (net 31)))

